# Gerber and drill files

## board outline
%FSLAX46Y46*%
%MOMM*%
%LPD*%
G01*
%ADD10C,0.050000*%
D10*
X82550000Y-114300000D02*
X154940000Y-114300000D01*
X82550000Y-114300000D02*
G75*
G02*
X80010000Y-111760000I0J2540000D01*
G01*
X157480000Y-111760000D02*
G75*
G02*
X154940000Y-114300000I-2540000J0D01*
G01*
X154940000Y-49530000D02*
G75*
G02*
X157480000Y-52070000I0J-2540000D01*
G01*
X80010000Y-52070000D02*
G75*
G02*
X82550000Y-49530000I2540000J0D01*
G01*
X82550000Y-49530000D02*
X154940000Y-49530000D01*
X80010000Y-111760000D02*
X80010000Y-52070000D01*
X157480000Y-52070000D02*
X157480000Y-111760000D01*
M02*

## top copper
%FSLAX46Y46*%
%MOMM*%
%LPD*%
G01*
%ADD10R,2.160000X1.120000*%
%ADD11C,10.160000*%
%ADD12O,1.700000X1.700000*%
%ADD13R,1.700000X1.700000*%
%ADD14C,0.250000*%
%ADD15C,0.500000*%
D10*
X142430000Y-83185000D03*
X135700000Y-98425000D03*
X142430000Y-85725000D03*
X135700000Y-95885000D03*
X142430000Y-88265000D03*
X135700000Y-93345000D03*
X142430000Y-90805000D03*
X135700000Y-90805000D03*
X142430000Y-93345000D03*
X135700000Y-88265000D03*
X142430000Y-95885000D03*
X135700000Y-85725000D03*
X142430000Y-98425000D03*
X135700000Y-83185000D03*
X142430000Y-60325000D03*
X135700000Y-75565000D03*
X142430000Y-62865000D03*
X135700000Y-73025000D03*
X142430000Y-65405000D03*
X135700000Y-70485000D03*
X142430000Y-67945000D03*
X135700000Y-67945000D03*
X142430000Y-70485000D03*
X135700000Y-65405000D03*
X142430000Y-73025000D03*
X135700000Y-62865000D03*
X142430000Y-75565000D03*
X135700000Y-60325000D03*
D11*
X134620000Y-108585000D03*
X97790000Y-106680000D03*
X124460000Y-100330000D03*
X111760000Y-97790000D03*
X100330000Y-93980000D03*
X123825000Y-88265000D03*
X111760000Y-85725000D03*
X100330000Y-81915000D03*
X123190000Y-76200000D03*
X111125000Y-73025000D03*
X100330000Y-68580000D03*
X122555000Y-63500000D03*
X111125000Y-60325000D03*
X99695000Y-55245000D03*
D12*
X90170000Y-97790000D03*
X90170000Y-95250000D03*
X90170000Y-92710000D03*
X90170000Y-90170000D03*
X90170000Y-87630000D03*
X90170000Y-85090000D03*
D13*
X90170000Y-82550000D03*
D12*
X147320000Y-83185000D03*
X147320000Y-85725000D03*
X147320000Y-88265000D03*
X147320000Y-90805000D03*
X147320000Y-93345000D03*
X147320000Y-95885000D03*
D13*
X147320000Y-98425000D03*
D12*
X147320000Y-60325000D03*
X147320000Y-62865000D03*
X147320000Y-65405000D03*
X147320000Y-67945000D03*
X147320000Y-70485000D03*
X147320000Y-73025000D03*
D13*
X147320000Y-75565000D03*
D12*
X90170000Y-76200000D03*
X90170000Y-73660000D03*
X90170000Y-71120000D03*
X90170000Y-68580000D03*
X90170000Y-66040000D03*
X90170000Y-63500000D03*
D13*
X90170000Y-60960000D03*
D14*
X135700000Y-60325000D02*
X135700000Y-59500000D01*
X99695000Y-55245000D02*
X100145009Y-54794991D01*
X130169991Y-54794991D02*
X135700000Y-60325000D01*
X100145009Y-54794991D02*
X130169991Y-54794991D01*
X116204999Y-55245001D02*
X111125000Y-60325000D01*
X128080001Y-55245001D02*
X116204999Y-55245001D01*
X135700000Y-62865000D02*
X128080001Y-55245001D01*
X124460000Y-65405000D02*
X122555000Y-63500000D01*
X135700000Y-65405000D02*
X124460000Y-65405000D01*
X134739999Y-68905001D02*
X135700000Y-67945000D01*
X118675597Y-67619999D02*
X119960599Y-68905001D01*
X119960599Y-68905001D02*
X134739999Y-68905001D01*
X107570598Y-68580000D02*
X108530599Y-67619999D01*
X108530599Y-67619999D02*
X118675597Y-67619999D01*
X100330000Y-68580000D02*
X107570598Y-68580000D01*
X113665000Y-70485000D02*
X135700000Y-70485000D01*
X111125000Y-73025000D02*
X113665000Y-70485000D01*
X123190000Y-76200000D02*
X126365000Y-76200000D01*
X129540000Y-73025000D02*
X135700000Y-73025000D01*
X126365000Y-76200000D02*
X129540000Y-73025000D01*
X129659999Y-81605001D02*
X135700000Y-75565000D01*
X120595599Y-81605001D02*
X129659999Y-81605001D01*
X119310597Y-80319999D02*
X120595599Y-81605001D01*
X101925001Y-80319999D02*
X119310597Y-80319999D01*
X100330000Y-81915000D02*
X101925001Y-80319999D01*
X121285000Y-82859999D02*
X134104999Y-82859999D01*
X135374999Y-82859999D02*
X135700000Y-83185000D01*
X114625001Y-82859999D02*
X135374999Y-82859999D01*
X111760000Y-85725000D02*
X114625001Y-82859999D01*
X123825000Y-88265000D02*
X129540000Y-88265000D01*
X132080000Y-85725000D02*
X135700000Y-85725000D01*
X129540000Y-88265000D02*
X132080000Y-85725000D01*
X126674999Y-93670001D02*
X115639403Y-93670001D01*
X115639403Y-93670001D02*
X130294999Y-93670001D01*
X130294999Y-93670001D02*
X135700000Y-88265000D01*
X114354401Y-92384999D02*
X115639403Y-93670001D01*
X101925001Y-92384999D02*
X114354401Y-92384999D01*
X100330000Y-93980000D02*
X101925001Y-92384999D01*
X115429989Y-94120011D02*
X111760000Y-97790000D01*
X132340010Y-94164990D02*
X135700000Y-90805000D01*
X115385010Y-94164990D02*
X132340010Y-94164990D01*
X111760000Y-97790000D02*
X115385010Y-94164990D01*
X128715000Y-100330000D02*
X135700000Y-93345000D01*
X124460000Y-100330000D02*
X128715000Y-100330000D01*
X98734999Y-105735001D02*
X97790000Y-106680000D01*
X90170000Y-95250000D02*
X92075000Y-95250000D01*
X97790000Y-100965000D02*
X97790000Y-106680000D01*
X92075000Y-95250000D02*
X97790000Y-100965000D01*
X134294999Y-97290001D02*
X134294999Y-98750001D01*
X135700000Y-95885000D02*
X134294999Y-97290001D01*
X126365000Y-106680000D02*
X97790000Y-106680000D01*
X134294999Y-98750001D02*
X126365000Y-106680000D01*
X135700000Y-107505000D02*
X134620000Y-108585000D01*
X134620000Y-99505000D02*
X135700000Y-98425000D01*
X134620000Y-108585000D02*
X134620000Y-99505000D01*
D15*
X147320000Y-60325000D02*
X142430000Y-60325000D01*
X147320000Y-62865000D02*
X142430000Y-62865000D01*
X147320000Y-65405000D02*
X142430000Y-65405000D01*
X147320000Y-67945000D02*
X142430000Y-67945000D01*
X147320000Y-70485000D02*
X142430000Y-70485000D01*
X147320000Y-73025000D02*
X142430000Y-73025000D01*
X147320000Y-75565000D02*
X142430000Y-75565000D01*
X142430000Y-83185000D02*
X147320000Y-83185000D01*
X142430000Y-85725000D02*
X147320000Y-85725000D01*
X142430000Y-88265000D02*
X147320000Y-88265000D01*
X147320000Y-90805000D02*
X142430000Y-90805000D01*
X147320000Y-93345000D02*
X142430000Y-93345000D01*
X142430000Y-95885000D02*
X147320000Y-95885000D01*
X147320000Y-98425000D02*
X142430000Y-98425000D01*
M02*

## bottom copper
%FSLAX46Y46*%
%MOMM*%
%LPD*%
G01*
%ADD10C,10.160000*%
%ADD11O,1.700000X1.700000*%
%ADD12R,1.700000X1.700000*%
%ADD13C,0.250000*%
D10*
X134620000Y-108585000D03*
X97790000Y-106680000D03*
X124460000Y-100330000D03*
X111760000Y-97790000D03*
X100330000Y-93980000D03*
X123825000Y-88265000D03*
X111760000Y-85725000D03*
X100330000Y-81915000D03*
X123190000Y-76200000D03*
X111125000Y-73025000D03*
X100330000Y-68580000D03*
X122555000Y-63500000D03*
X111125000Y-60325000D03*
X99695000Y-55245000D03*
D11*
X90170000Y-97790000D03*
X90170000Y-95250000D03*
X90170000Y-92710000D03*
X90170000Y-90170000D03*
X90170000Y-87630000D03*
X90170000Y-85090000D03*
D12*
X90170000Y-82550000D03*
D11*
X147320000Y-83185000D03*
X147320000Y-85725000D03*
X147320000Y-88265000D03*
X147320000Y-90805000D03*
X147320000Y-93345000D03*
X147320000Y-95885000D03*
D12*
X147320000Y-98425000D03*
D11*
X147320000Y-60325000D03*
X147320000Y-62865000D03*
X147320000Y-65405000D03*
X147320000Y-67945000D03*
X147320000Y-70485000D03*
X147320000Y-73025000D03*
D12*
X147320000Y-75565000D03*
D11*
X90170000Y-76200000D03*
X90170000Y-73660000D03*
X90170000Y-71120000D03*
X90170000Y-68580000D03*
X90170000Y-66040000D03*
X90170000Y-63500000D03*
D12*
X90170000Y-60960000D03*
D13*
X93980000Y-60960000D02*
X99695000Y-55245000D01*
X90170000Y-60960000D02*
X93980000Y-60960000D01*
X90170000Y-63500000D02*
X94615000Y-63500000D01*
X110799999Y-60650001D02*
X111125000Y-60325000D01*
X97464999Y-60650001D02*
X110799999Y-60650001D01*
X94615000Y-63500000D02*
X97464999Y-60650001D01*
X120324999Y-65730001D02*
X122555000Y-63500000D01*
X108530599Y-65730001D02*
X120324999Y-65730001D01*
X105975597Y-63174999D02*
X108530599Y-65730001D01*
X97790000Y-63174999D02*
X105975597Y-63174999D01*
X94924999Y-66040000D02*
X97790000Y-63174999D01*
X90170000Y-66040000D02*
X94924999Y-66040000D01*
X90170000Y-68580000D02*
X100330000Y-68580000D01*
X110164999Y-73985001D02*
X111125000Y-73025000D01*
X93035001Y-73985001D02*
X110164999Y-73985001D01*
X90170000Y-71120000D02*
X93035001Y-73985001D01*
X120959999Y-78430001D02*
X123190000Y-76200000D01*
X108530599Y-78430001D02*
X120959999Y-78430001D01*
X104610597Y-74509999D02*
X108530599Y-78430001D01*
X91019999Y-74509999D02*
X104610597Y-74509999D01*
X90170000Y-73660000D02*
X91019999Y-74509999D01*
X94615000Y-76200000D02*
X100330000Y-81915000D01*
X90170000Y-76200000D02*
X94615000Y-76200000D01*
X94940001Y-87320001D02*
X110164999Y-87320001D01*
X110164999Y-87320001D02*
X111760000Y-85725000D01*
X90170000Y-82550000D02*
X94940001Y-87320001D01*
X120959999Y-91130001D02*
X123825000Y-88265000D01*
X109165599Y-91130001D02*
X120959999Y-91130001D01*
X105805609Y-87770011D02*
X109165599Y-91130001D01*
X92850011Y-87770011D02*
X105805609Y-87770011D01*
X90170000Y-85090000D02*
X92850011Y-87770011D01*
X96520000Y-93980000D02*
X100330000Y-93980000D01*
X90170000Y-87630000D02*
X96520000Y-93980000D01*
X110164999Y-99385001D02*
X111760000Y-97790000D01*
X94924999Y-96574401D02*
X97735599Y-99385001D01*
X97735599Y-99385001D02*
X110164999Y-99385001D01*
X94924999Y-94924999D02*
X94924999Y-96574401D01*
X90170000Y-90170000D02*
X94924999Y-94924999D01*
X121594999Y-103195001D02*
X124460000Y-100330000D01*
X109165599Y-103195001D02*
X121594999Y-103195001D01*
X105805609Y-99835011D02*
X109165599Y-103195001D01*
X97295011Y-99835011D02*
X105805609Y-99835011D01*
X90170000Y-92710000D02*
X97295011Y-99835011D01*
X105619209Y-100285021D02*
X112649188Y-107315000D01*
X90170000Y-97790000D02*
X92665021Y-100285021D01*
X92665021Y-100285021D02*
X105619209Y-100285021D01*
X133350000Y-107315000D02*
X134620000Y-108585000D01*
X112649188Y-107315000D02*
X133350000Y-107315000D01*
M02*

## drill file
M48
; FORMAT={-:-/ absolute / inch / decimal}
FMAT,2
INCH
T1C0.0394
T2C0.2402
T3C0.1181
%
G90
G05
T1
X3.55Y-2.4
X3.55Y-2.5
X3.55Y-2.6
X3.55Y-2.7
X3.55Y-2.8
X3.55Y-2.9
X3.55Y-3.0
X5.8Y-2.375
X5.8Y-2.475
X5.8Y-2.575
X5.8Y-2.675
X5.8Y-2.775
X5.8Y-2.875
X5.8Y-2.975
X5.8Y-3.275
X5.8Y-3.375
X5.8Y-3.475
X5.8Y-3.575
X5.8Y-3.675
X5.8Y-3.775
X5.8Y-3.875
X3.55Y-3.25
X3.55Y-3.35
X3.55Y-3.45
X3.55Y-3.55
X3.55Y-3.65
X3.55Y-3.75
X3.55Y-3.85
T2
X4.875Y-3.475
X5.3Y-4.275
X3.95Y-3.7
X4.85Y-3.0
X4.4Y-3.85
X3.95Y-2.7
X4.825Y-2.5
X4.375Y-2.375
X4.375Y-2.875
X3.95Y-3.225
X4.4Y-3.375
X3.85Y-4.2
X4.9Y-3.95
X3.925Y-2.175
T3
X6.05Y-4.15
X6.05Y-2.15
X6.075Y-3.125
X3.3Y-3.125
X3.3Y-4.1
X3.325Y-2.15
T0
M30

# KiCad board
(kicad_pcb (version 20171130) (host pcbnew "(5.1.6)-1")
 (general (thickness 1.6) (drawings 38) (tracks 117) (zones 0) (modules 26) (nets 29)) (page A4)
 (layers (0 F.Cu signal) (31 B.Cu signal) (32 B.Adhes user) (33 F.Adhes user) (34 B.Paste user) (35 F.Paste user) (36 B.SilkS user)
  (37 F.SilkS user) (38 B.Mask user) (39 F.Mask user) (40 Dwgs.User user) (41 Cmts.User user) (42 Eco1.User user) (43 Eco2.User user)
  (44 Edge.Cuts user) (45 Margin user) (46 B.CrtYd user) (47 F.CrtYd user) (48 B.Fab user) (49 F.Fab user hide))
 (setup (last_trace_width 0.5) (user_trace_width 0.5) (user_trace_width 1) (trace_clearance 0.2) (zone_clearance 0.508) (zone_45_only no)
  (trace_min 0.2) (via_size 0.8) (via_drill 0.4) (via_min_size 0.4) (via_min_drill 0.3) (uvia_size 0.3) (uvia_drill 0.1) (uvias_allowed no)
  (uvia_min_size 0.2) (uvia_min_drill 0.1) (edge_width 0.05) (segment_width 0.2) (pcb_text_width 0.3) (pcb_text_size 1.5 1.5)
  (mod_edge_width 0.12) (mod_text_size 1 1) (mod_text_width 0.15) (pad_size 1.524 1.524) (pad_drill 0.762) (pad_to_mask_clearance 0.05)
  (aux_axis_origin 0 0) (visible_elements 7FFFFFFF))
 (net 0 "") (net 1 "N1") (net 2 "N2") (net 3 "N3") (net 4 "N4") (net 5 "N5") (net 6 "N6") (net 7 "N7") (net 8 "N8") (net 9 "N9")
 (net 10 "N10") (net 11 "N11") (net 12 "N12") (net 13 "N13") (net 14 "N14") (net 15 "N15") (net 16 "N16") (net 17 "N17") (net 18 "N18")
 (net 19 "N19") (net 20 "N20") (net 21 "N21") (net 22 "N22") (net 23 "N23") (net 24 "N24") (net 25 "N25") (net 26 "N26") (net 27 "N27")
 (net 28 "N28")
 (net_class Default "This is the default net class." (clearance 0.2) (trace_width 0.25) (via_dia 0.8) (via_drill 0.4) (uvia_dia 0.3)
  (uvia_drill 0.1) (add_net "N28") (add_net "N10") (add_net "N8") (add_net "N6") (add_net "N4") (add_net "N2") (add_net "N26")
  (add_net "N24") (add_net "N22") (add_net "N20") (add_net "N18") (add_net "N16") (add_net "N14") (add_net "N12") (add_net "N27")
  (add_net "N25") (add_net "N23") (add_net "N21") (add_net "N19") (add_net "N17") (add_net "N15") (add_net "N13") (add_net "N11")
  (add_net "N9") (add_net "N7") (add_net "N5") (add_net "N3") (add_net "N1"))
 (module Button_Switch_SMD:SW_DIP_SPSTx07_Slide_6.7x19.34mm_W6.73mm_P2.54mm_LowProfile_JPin (layer F.Cu) (at 139.065 90.805)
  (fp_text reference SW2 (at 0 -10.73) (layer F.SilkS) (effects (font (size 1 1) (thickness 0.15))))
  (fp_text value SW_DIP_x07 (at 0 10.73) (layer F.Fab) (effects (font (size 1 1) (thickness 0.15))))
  (pad 14 smd rect (at 3.365 -7.62) (size 2.16 1.12) (layers F.Cu F.Paste F.Mask) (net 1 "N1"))
  (pad 7 smd rect (at -3.365 7.62) (size 2.16 1.12) (layers F.Cu F.Paste F.Mask) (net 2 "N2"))
  (pad 13 smd rect (at 3.365 -5.08) (size 2.16 1.12) (layers F.Cu F.Paste F.Mask) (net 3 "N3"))
  (pad 6 smd rect (at -3.365 5.08) (size 2.16 1.12) (layers F.Cu F.Paste F.Mask) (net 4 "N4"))
  (pad 12 smd rect (at 3.365 -2.54) (size 2.16 1.12) (layers F.Cu F.Paste F.Mask) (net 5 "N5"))
  (pad 5 smd rect (at -3.365 2.54) (size 2.16 1.12) (layers F.Cu F.Paste F.Mask) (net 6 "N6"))
  (pad 11 smd rect (at 3.365 0) (size 2.16 1.12) (layers F.Cu F.Paste F.Mask) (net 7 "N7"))
  (pad 4 smd rect (at -3.365 0) (size 2.16 1.12) (layers F.Cu F.Paste F.Mask) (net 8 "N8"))
  (pad 10 smd rect (at 3.365 2.54) (size 2.16 1.12) (layers F.Cu F.Paste F.Mask) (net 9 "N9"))
  (pad 3 smd rect (at -3.365 -2.54) (size 2.16 1.12) (layers F.Cu F.Paste F.Mask) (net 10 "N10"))
  (pad 9 smd rect (at 3.365 5.08) (size 2.16 1.12) (layers F.Cu F.Paste F.Mask) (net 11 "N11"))
  (pad 2 smd rect (at -3.365 -5.08) (size 2.16 1.12) (layers F.Cu F.Paste F.Mask) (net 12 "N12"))
  (pad 8 smd rect (at 3.365 7.62) (size 2.16 1.12) (layers F.Cu F.Paste F.Mask) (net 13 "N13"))
  (pad 1 smd rect (at -3.365 -7.62) (size 2.16 1.12) (layers F.Cu F.Paste F.Mask) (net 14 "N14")))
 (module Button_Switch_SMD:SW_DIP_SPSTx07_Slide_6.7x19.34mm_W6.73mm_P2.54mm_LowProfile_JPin (layer F.Cu) (at 139.065 67.945)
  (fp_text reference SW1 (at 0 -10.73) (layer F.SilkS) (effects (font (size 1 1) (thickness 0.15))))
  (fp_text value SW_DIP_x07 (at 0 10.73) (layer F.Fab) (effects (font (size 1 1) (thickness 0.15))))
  (pad 14 smd rect (at 3.365 -7.62) (size 2.16 1.12) (layers F.Cu F.Paste F.Mask) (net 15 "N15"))
  (pad 7 smd rect (at -3.365 7.62) (size 2.16 1.12) (layers F.Cu F.Paste F.Mask) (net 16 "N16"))
  (pad 13 smd rect (at 3.365 -5.08) (size 2.16 1.12) (layers F.Cu F.Paste F.Mask) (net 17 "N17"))
  (pad 6 smd rect (at -3.365 5.08) (size 2.16 1.12) (layers F.Cu F.Paste F.Mask) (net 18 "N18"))
  (pad 12 smd rect (at 3.365 -2.54) (size 2.16 1.12) (layers F.Cu F.Paste F.Mask) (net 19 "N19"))
  (pad 5 smd rect (at -3.365 2.54) (size 2.16 1.12) (layers F.Cu F.Paste F.Mask) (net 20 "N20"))
  (pad 11 smd rect (at 3.365 0) (size 2.16 1.12) (layers F.Cu F.Paste F.Mask) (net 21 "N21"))
  (pad 4 smd rect (at -3.365 0) (size 2.16 1.12) (layers F.Cu F.Paste F.Mask) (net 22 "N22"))
  (pad 10 smd rect (at 3.365 2.54) (size 2.16 1.12) (layers F.Cu F.Paste F.Mask) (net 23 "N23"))
  (pad 3 smd rect (at -3.365 -2.54) (size 2.16 1.12) (layers F.Cu F.Paste F.Mask) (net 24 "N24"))
  (pad 9 smd rect (at 3.365 5.08) (size 2.16 1.12) (layers F.Cu F.Paste F.Mask) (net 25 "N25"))
  (pad 2 smd rect (at -3.365 -5.08) (size 2.16 1.12) (layers F.Cu F.Paste F.Mask) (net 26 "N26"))
  (pad 8 smd rect (at 3.365 7.62) (size 2.16 1.12) (layers F.Cu F.Paste F.Mask) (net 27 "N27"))
  (pad 1 smd rect (at -3.365 -7.62) (size 2.16 1.12) (layers F.Cu F.Paste F.Mask) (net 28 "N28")))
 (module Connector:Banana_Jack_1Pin (layer F.Cu) (at 134.62 108.585)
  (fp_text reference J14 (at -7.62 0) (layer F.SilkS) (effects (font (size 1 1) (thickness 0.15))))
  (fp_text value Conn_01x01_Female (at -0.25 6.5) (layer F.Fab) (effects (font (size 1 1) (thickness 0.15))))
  (pad 1 thru_hole circle (at 0 0) (size 10.16 10.16) (drill 6.1) (layers *.Cu *.Mask) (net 2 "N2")))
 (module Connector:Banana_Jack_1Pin (layer F.Cu) (at 97.79 106.68)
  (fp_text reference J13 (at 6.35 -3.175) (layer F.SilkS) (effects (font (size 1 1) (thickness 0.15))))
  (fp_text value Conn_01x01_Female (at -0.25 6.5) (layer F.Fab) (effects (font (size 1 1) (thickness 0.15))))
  (pad 1 thru_hole circle (at 0 0) (size 10.16 10.16) (drill 6.1) (layers *.Cu *.Mask) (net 4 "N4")))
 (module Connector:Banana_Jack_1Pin (layer F.Cu) (at 124.46 100.33)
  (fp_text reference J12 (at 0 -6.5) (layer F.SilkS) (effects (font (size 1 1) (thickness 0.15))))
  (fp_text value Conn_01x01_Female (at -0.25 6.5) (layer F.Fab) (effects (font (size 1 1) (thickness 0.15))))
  (pad 1 thru_hole circle (at 0 0) (size 10.16 10.16) (drill 6.1) (layers *.Cu *.Mask) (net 6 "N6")))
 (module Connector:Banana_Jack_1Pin (layer F.Cu) (at 111.76 97.79)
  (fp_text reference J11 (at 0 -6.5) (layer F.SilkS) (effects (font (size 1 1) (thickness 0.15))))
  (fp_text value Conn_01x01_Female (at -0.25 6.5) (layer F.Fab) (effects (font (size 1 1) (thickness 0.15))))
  (pad 1 thru_hole circle (at 0 0) (size 10.16 10.16) (drill 6.1) (layers *.Cu *.Mask) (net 8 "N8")))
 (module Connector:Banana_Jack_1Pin (layer F.Cu) (at 100.33 93.98)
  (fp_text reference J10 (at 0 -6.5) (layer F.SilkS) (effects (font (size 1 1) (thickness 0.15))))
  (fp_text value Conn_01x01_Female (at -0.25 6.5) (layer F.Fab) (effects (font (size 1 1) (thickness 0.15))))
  (pad 1 thru_hole circle (at 0 0) (size 10.16 10.16) (drill 6.1) (layers *.Cu *.Mask) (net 10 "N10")))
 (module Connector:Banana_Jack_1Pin (layer F.Cu) (at 123.825 88.265)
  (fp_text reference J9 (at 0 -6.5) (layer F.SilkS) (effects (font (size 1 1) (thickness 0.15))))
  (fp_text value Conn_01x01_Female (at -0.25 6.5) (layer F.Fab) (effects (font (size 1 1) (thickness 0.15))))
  (pad 1 thru_hole circle (at 0 0) (size 10.16 10.16) (drill 6.1) (layers *.Cu *.Mask) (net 12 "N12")))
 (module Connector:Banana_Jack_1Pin (layer F.Cu) (at 111.76 85.725)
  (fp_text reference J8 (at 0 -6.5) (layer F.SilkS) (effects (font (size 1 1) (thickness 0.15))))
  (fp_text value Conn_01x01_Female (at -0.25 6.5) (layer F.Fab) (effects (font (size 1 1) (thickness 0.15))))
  (pad 1 thru_hole circle (at 0 0) (size 10.16 10.16) (drill 6.1) (layers *.Cu *.Mask) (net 14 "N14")))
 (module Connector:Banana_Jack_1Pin (layer F.Cu) (at 100.33 81.915)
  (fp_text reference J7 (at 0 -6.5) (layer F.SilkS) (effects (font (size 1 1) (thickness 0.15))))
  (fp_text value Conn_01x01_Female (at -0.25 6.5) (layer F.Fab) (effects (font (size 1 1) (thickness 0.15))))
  (pad 1 thru_hole circle (at 0 0) (size 10.16 10.16) (drill 6.1) (layers *.Cu *.Mask) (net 16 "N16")))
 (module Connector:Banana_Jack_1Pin (layer F.Cu) (at 123.19 76.2)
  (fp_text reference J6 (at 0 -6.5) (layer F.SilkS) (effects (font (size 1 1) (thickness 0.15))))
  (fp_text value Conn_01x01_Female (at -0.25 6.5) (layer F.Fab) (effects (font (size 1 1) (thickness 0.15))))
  (pad 1 thru_hole circle (at 0 0) (size 10.16 10.16) (drill 6.1) (layers *.Cu *.Mask) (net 18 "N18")))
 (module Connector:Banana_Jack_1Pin (layer F.Cu) (at 111.125 73.025)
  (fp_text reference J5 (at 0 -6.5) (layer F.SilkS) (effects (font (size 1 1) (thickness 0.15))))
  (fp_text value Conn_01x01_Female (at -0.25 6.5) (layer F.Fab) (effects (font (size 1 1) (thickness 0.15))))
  (pad 1 thru_hole circle (at 0 0) (size 10.16 10.16) (drill 6.1) (layers *.Cu *.Mask) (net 20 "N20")))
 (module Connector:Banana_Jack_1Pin (layer F.Cu) (at 100.33 68.58)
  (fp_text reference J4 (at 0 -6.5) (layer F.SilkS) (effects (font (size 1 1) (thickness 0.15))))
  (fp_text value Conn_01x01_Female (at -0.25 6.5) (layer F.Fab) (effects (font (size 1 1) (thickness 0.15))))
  (pad 1 thru_hole circle (at 0 0) (size 10.16 10.16) (drill 6.1) (layers *.Cu *.Mask) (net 22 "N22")))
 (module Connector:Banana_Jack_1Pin (layer F.Cu) (at 122.555 63.5)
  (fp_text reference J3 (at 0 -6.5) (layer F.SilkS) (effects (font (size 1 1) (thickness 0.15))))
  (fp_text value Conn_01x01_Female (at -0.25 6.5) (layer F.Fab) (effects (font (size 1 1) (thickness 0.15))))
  (pad 1 thru_hole circle (at 0 0) (size 10.16 10.16) (drill 6.1) (layers *.Cu *.Mask) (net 24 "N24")))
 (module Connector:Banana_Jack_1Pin (layer F.Cu) (at 111.125 60.325)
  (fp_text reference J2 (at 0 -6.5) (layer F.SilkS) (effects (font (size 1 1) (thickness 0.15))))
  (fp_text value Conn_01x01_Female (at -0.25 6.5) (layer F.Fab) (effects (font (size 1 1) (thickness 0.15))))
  (pad 1 thru_hole circle (at 0 0) (size 10.16 10.16) (drill 6.1) (layers *.Cu *.Mask) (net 26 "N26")))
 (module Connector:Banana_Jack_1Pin (layer F.Cu) (at 99.695 55.245)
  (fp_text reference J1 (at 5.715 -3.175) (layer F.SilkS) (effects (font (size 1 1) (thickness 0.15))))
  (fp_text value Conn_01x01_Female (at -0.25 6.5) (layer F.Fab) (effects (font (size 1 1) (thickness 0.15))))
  (pad 1 thru_hole circle (at 0 0) (size 10.16 10.16) (drill 6.1) (layers *.Cu *.Mask) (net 28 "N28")))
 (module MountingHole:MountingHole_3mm (layer F.Cu) (at 83.82 104.14)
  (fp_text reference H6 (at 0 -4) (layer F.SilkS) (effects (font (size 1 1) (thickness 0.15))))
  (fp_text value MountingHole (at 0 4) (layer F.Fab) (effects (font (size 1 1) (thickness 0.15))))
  (pad 1 np_thru_hole circle (at 0 0) (size 3 3) (drill 3) (layers *.Cu *.Mask)))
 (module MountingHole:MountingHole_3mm (layer F.Cu) (at 153.67 54.61)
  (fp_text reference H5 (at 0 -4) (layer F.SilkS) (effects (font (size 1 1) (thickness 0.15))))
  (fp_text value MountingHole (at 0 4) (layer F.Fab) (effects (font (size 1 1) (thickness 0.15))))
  (pad 1 np_thru_hole circle (at 0 0) (size 3 3) (drill 3) (layers *.Cu *.Mask)))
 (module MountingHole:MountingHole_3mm (layer F.Cu) (at 154.305 79.375)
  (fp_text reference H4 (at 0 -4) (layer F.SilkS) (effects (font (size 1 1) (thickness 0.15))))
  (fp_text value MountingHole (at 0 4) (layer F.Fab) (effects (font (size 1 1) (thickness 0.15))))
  (pad 1 np_thru_hole circle (at 0 0) (size 3 3) (drill 3) (layers *.Cu *.Mask)))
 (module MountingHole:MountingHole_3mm (layer F.Cu) (at 153.67 105.41)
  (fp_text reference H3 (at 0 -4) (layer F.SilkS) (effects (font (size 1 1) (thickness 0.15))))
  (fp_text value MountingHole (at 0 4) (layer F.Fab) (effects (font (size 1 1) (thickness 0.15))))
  (pad 1 np_thru_hole circle (at 0 0) (size 3 3) (drill 3) (layers *.Cu *.Mask)))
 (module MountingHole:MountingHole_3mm (layer F.Cu) (at 83.82 79.375)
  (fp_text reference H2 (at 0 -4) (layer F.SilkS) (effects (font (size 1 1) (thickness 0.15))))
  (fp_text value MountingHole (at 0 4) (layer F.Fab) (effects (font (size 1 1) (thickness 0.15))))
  (pad 1 np_thru_hole circle (at 0 0) (size 3 3) (drill 3) (layers *.Cu *.Mask)))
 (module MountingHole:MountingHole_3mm (layer F.Cu) (at 84.455 54.61)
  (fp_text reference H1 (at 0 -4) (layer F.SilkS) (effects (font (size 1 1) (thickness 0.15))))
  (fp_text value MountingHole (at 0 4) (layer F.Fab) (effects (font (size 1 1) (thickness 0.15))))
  (pad 1 np_thru_hole circle (at 0 0) (size 3 3) (drill 3) (layers *.Cu *.Mask)))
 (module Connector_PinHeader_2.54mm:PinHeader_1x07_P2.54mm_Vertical (layer F.Cu) (at 90.17 82.55)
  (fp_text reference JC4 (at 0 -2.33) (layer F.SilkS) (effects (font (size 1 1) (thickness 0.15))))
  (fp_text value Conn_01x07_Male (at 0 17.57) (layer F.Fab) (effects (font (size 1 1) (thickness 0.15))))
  (pad 7 thru_hole oval (at 0 15.24) (size 1.7 1.7) (drill 1) (layers *.Cu *.Mask) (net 2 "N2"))
  (pad 6 thru_hole oval (at 0 12.7) (size 1.7 1.7) (drill 1) (layers *.Cu *.Mask) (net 4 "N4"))
  (pad 5 thru_hole oval (at 0 10.16) (size 1.7 1.7) (drill 1) (layers *.Cu *.Mask) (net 6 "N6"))
  (pad 4 thru_hole oval (at 0 7.62) (size 1.7 1.7) (drill 1) (layers *.Cu *.Mask) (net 8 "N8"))
  (pad 3 thru_hole oval (at 0 5.08) (size 1.7 1.7) (drill 1) (layers *.Cu *.Mask) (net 10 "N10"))
  (pad 2 thru_hole oval (at 0 2.54) (size 1.7 1.7) (drill 1) (layers *.Cu *.Mask) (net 12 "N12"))
  (pad 1 thru_hole rect (at 0 0) (size 1.7 1.7) (drill 1) (layers *.Cu *.Mask) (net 14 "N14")))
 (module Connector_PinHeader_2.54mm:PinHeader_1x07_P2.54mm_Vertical (layer F.Cu) (at 147.32 98.425 180)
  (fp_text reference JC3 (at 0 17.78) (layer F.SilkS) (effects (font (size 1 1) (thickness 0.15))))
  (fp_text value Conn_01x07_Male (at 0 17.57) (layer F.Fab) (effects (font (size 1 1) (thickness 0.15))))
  (pad 7 thru_hole oval (at 0 15.24 180) (size 1.7 1.7) (drill 1) (layers *.Cu *.Mask) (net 1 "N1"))
  (pad 6 thru_hole oval (at 0 12.7 180) (size 1.7 1.7) (drill 1) (layers *.Cu *.Mask) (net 3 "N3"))
  (pad 5 thru_hole oval (at 0 10.16 180) (size 1.7 1.7) (drill 1) (layers *.Cu *.Mask) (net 5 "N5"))
  (pad 4 thru_hole oval (at 0 7.62 180) (size 1.7 1.7) (drill 1) (layers *.Cu *.Mask) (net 7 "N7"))
  (pad 3 thru_hole oval (at 0 5.08 180) (size 1.7 1.7) (drill 1) (layers *.Cu *.Mask) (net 9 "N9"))
  (pad 2 thru_hole oval (at 0 2.54 180) (size 1.7 1.7) (drill 1) (layers *.Cu *.Mask) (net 11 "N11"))
  (pad 1 thru_hole rect (at 0 0 180) (size 1.7 1.7) (drill 1) (layers *.Cu *.Mask) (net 13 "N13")))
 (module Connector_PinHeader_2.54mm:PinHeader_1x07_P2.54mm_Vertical (layer F.Cu) (at 147.32 75.565 180)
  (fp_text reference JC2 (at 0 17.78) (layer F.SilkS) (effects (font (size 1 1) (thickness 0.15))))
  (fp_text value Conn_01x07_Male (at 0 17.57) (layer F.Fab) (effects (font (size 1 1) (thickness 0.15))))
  (pad 7 thru_hole oval (at 0 15.24 180) (size 1.7 1.7) (drill 1) (layers *.Cu *.Mask) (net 15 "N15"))
  (pad 6 thru_hole oval (at 0 12.7 180) (size 1.7 1.7) (drill 1) (layers *.Cu *.Mask) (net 17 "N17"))
  (pad 5 thru_hole oval (at 0 10.16 180) (size 1.7 1.7) (drill 1) (layers *.Cu *.Mask) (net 19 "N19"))
  (pad 4 thru_hole oval (at 0 7.62 180) (size 1.7 1.7) (drill 1) (layers *.Cu *.Mask) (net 21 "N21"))
  (pad 3 thru_hole oval (at 0 5.08 180) (size 1.7 1.7) (drill 1) (layers *.Cu *.Mask) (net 23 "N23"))
  (pad 2 thru_hole oval (at 0 2.54 180) (size 1.7 1.7) (drill 1) (layers *.Cu *.Mask) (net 25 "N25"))
  (pad 1 thru_hole rect (at 0 0 180) (size 1.7 1.7) (drill 1) (layers *.Cu *.Mask) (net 27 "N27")))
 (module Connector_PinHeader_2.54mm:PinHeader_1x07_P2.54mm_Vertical (layer F.Cu) (at 90.17 60.96)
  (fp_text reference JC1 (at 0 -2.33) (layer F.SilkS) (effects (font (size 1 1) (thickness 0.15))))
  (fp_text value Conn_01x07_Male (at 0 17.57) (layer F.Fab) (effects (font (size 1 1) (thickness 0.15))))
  (pad 7 thru_hole oval (at 0 15.24) (size 1.7 1.7) (drill 1) (layers *.Cu *.Mask) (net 16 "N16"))
  (pad 6 thru_hole oval (at 0 12.7) (size 1.7 1.7) (drill 1) (layers *.Cu *.Mask) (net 18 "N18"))
  (pad 5 thru_hole oval (at 0 10.16) (size 1.7 1.7) (drill 1) (layers *.Cu *.Mask) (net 20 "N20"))
  (pad 4 thru_hole oval (at 0 7.62) (size 1.7 1.7) (drill 1) (layers *.Cu *.Mask) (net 22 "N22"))
  (pad 3 thru_hole oval (at 0 5.08) (size 1.7 1.7) (drill 1) (layers *.Cu *.Mask) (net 24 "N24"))
  (pad 2 thru_hole oval (at 0 2.54) (size 1.7 1.7) (drill 1) (layers *.Cu *.Mask) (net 26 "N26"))
  (pad 1 thru_hole rect (at 0 0) (size 1.7 1.7) (drill 1) (layers *.Cu *.Mask) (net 28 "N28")))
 (gr_line (start 82.55 114.3) (end 154.94 114.3) (layer Edge.Cuts) (width 0.05))
 (gr_arc (start 82.55 111.76) (end 80.01 111.76) (angle -90) (layer Edge.Cuts) (width 0.05))
 (gr_arc (start 154.94 111.76) (end 154.94 114.3) (angle -90) (layer Edge.Cuts) (width 0.05))
 (gr_arc (start 154.94 52.07) (end 157.48 52.07) (angle -90) (layer Edge.Cuts) (width 0.05))
 (gr_arc (start 82.55 52.07) (end 82.55 49.53) (angle -90) (layer Edge.Cuts) (width 0.05))
 (gr_line (start 82.55 49.53) (end 154.94 49.53) (layer Edge.Cuts) (width 0.05))
 (gr_line (start 80.01 111.76) (end 80.01 52.07) (layer Edge.Cuts) (width 0.05))
 (gr_line (start 157.48 52.07) (end 157.48 111.76) (layer Edge.Cuts) (width 0.05))
 (segment (start 135.7 60.325) (end 135.7 59.5) (width 0.25) (layer F.Cu) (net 28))
 (segment (start 93.98 60.96) (end 99.695 55.245) (width 0.25) (layer B.Cu) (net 28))
 (segment (start 90.17 60.96) (end 93.98 60.96) (width 0.25) (layer B.Cu) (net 28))
 (segment (start 99.695 55.245) (end 100.145009 54.794991) (width 0.25) (layer F.Cu) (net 28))
 (segment (start 130.169991 54.794991) (end 135.7 60.325) (width 0.25) (layer F.Cu) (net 28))
 (segment (start 100.145009 54.794991) (end 130.169991 54.794991) (width 0.25) (layer F.Cu) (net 28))
 (segment (start 116.204999 55.245001) (end 111.125 60.325) (width 0.25) (layer F.Cu) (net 26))
 (segment (start 128.080001 55.245001) (end 116.204999 55.245001) (width 0.25) (layer F.Cu) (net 26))
 (segment (start 135.7 62.865) (end 128.080001 55.245001) (width 0.25) (layer F.Cu) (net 26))
 (segment (start 90.17 63.5) (end 94.615 63.5) (width 0.25) (layer B.Cu) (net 26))
 (segment (start 110.799999 60.650001) (end 111.125 60.325) (width 0.25) (layer B.Cu) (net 26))
 (segment (start 97.464999 60.650001) (end 110.799999 60.650001) (width 0.25) (layer B.Cu) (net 26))
 (segment (start 94.615 63.5) (end 97.464999 60.650001) (width 0.25) (layer B.Cu) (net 26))
 (segment (start 124.46 65.405) (end 122.555 63.5) (width 0.25) (layer F.Cu) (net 24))
 (segment (start 135.7 65.405) (end 124.46 65.405) (width 0.25) (layer F.Cu) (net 24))
 (segment (start 120.324999 65.730001) (end 122.555 63.5) (width 0.25) (layer B.Cu) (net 24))
 (segment (start 108.530599 65.730001) (end 120.324999 65.730001) (width 0.25) (layer B.Cu) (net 24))
 (segment (start 105.975597 63.174999) (end 108.530599 65.730001) (width 0.25) (layer B.Cu) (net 24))
 (segment (start 97.79 63.174999) (end 105.975597 63.174999) (width 0.25) (layer B.Cu) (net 24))
 (segment (start 94.924999 66.04) (end 97.79 63.174999) (width 0.25) (layer B.Cu) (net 24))
 (segment (start 90.17 66.04) (end 94.924999 66.04) (width 0.25) (layer B.Cu) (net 24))
 (segment (start 134.739999 68.905001) (end 135.7 67.945) (width 0.25) (layer F.Cu) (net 22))
 (segment (start 118.675597 67.619999) (end 119.960599 68.905001) (width 0.25) (layer F.Cu) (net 22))
 (segment (start 119.960599 68.905001) (end 134.739999 68.905001) (width 0.25) (layer F.Cu) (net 22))
 (segment (start 107.570598 68.58) (end 108.530599 67.619999) (width 0.25) (layer F.Cu) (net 22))
 (segment (start 108.530599 67.619999) (end 118.675597 67.619999) (width 0.25) (layer F.Cu) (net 22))
 (segment (start 100.33 68.58) (end 107.570598 68.58) (width 0.25) (layer F.Cu) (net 22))
 (segment (start 90.17 68.58) (end 100.33 68.58) (width 0.25) (layer B.Cu) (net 22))
 (segment (start 113.665 70.485) (end 135.7 70.485) (width 0.25) (layer F.Cu) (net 20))
 (segment (start 111.125 73.025) (end 113.665 70.485) (width 0.25) (layer F.Cu) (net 20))
 (segment (start 110.164999 73.985001) (end 111.125 73.025) (width 0.25) (layer B.Cu) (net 20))
 (segment (start 93.035001 73.985001) (end 110.164999 73.985001) (width 0.25) (layer B.Cu) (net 20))
 (segment (start 90.17 71.12) (end 93.035001 73.985001) (width 0.25) (layer B.Cu) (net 20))
 (segment (start 123.19 76.2) (end 126.365 76.2) (width 0.25) (layer F.Cu) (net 18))
 (segment (start 129.54 73.025) (end 135.7 73.025) (width 0.25) (layer F.Cu) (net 18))
 (segment (start 126.365 76.2) (end 129.54 73.025) (width 0.25) (layer F.Cu) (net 18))
 (segment (start 120.959999 78.430001) (end 123.19 76.2) (width 0.25) (layer B.Cu) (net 18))
 (segment (start 108.530599 78.430001) (end 120.959999 78.430001) (width 0.25) (layer B.Cu) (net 18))
 (segment (start 104.610597 74.509999) (end 108.530599 78.430001) (width 0.25) (layer B.Cu) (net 18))
 (segment (start 91.019999 74.509999) (end 104.610597 74.509999) (width 0.25) (layer B.Cu) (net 18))
 (segment (start 90.17 73.66) (end 91.019999 74.509999) (width 0.25) (layer B.Cu) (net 18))
 (segment (start 94.615 76.2) (end 100.33 81.915) (width 0.25) (layer B.Cu) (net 16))
 (segment (start 90.17 76.2) (end 94.615 76.2) (width 0.25) (layer B.Cu) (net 16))
 (segment (start 129.659999 81.605001) (end 135.7 75.565) (width 0.25) (layer F.Cu) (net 16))
 (segment (start 120.595599 81.605001) (end 129.659999 81.605001) (width 0.25) (layer F.Cu) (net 16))
 (segment (start 119.310597 80.319999) (end 120.595599 81.605001) (width 0.25) (layer F.Cu) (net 16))
 (segment (start 101.925001 80.319999) (end 119.310597 80.319999) (width 0.25) (layer F.Cu) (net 16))
 (segment (start 100.33 81.915) (end 101.925001 80.319999) (width 0.25) (layer F.Cu) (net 16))
 (segment (start 121.285 82.859999) (end 134.104999 82.859999) (width 0.25) (layer F.Cu) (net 14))
 (segment (start 94.940001 87.320001) (end 110.164999 87.320001) (width 0.25) (layer B.Cu) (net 14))
 (segment (start 110.164999 87.320001) (end 111.76 85.725) (width 0.25) (layer B.Cu) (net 14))
 (segment (start 90.17 82.55) (end 94.940001 87.320001) (width 0.25) (layer B.Cu) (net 14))
 (segment (start 135.374999 82.859999) (end 135.7 83.185) (width 0.25) (layer F.Cu) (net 14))
 (segment (start 114.625001 82.859999) (end 135.374999 82.859999) (width 0.25) (layer F.Cu) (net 14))
 (segment (start 111.76 85.725) (end 114.625001 82.859999) (width 0.25) (layer F.Cu) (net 14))
 (segment (start 120.959999 91.130001) (end 123.825 88.265) (width 0.25) (layer B.Cu) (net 12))
 (segment (start 109.165599 91.130001) (end 120.959999 91.130001) (width 0.25) (layer B.Cu) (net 12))
 (segment (start 105.805609 87.770011) (end 109.165599 91.130001) (width 0.25) (layer B.Cu) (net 12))
 (segment (start 92.850011 87.770011) (end 105.805609 87.770011) (width 0.25) (layer B.Cu) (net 12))
 (segment (start 90.17 85.09) (end 92.850011 87.770011) (width 0.25) (layer B.Cu) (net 12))
 (segment (start 123.825 88.265) (end 129.54 88.265) (width 0.25) (layer F.Cu) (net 12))
 (segment (start 132.08 85.725) (end 135.7 85.725) (width 0.25) (layer F.Cu) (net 12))
 (segment (start 129.54 88.265) (end 132.08 85.725) (width 0.25) (layer F.Cu) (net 12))
 (segment (start 126.674999 93.670001) (end 115.639403 93.670001) (width 0.25) (layer F.Cu) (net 10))
 (segment (start 96.52 93.98) (end 100.33 93.98) (width 0.25) (layer B.Cu) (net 10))
 (segment (start 90.17 87.63) (end 96.52 93.98) (width 0.25) (layer B.Cu) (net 10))
 (segment (start 115.639403 93.670001) (end 130.294999 93.670001) (width 0.25) (layer F.Cu) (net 10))
 (segment (start 130.294999 93.670001) (end 135.7 88.265) (width 0.25) (layer F.Cu) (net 10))
 (segment (start 114.354401 92.384999) (end 115.639403 93.670001) (width 0.25) (layer F.Cu) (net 10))
 (segment (start 101.925001 92.384999) (end 114.354401 92.384999) (width 0.25) (layer F.Cu) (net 10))
 (segment (start 100.33 93.98) (end 101.925001 92.384999) (width 0.25) (layer F.Cu) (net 10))
 (segment (start 115.429989 94.120011) (end 111.76 97.79) (width 0.25) (layer F.Cu) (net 8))
 (segment (start 110.164999 99.385001) (end 111.76 97.79) (width 0.25) (layer B.Cu) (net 8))
 (segment (start 94.924999 96.574401) (end 97.735599 99.385001) (width 0.25) (layer B.Cu) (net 8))
 (segment (start 97.735599 99.385001) (end 110.164999 99.385001) (width 0.25) (layer B.Cu) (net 8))
 (segment (start 94.924999 94.924999) (end 94.924999 96.574401) (width 0.25) (layer B.Cu) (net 8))
 (segment (start 90.17 90.17) (end 94.924999 94.924999) (width 0.25) (layer B.Cu) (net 8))
 (segment (start 132.34001 94.16499) (end 135.7 90.805) (width 0.25) (layer F.Cu) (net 8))
 (segment (start 115.38501 94.16499) (end 132.34001 94.16499) (width 0.25) (layer F.Cu) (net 8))
 (segment (start 111.76 97.79) (end 115.38501 94.16499) (width 0.25) (layer F.Cu) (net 8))
 (segment (start 121.594999 103.195001) (end 124.46 100.33) (width 0.25) (layer B.Cu) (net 6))
 (segment (start 109.165599 103.195001) (end 121.594999 103.195001) (width 0.25) (layer B.Cu) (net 6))
 (segment (start 105.805609 99.835011) (end 109.165599 103.195001) (width 0.25) (layer B.Cu) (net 6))
 (segment (start 97.295011 99.835011) (end 105.805609 99.835011) (width 0.25) (layer B.Cu) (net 6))
 (segment (start 90.17 92.71) (end 97.295011 99.835011) (width 0.25) (layer B.Cu) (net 6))
 (segment (start 128.715 100.33) (end 135.7 93.345) (width 0.25) (layer F.Cu) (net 6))
 (segment (start 124.46 100.33) (end 128.715 100.33) (width 0.25) (layer F.Cu) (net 6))
 (segment (start 98.734999 105.735001) (end 97.79 106.68) (width 0.25) (layer F.Cu) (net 4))
 (segment (start 90.17 95.25) (end 92.075 95.25) (width 0.25) (layer F.Cu) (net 4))
 (segment (start 97.79 100.965) (end 97.79 106.68) (width 0.25) (layer F.Cu) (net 4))
 (segment (start 92.075 95.25) (end 97.79 100.965) (width 0.25) (layer F.Cu) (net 4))
 (segment (start 134.294999 97.290001) (end 134.294999 98.750001) (width 0.25) (layer F.Cu) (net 4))
 (segment (start 135.7 95.885) (end 134.294999 97.290001) (width 0.25) (layer F.Cu) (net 4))
 (segment (start 126.365 106.68) (end 97.79 106.68) (width 0.25) (layer F.Cu) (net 4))
 (segment (start 134.294999 98.750001) (end 126.365 106.68) (width 0.25) (layer F.Cu) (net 4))
 (segment (start 135.7 107.505) (end 134.62 108.585) (width 0.25) (layer F.Cu) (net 2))
 (segment (start 105.619209 100.285021) (end 112.649188 107.315) (width 0.25) (layer B.Cu) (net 2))
 (segment (start 90.17 97.79) (end 92.665021 100.285021) (width 0.25) (layer B.Cu) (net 2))
 (segment (start 92.665021 100.285021) (end 105.619209 100.285021) (width 0.25) (layer B.Cu) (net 2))
 (segment (start 133.35 107.315) (end 134.62 108.585) (width 0.25) (layer B.Cu) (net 2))
 (segment (start 112.649188 107.315) (end 133.35 107.315) (width 0.25) (layer B.Cu) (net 2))
 (segment (start 134.62 99.505) (end 135.7 98.425) (width 0.25) (layer F.Cu) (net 2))
 (segment (start 134.62 108.585) (end 134.62 99.505) (width 0.25) (layer F.Cu) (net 2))
 (segment (start 147.32 60.325) (end 142.43 60.325) (width 0.5) (layer F.Cu) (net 15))
 (segment (start 147.32 62.865) (end 142.43 62.865) (width 0.5) (layer F.Cu) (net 17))
 (segment (start 147.32 65.405) (end 142.43 65.405) (width 0.5) (layer F.Cu) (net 19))
 (segment (start 147.32 67.945) (end 142.43 67.945) (width 0.5) (layer F.Cu) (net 21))
 (segment (start 147.32 70.485) (end 142.43 70.485) (width 0.5) (layer F.Cu) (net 23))
 (segment (start 147.32 73.025) (end 142.43 73.025) (width 0.5) (layer F.Cu) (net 25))
 (segment (start 147.32 75.565) (end 142.43 75.565) (width 0.5) (layer F.Cu) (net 27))
 (segment (start 142.43 83.185) (end 147.32 83.185) (width 0.5) (layer F.Cu) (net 1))
 (segment (start 142.43 85.725) (end 147.32 85.725) (width 0.5) (layer F.Cu) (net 3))
 (segment (start 142.43 88.265) (end 147.32 88.265) (width 0.5) (layer F.Cu) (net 5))
 (segment (start 147.32 90.805) (end 142.43 90.805) (width 0.5) (layer F.Cu) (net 7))
 (segment (start 147.32 93.345) (end 142.43 93.345) (width 0.5) (layer F.Cu) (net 9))
 (segment (start 142.43 95.885) (end 147.32 95.885) (width 0.5) (layer F.Cu) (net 11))
 (segment (start 147.32 98.425) (end 142.43 98.425) (width 0.5) (layer F.Cu) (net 13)))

